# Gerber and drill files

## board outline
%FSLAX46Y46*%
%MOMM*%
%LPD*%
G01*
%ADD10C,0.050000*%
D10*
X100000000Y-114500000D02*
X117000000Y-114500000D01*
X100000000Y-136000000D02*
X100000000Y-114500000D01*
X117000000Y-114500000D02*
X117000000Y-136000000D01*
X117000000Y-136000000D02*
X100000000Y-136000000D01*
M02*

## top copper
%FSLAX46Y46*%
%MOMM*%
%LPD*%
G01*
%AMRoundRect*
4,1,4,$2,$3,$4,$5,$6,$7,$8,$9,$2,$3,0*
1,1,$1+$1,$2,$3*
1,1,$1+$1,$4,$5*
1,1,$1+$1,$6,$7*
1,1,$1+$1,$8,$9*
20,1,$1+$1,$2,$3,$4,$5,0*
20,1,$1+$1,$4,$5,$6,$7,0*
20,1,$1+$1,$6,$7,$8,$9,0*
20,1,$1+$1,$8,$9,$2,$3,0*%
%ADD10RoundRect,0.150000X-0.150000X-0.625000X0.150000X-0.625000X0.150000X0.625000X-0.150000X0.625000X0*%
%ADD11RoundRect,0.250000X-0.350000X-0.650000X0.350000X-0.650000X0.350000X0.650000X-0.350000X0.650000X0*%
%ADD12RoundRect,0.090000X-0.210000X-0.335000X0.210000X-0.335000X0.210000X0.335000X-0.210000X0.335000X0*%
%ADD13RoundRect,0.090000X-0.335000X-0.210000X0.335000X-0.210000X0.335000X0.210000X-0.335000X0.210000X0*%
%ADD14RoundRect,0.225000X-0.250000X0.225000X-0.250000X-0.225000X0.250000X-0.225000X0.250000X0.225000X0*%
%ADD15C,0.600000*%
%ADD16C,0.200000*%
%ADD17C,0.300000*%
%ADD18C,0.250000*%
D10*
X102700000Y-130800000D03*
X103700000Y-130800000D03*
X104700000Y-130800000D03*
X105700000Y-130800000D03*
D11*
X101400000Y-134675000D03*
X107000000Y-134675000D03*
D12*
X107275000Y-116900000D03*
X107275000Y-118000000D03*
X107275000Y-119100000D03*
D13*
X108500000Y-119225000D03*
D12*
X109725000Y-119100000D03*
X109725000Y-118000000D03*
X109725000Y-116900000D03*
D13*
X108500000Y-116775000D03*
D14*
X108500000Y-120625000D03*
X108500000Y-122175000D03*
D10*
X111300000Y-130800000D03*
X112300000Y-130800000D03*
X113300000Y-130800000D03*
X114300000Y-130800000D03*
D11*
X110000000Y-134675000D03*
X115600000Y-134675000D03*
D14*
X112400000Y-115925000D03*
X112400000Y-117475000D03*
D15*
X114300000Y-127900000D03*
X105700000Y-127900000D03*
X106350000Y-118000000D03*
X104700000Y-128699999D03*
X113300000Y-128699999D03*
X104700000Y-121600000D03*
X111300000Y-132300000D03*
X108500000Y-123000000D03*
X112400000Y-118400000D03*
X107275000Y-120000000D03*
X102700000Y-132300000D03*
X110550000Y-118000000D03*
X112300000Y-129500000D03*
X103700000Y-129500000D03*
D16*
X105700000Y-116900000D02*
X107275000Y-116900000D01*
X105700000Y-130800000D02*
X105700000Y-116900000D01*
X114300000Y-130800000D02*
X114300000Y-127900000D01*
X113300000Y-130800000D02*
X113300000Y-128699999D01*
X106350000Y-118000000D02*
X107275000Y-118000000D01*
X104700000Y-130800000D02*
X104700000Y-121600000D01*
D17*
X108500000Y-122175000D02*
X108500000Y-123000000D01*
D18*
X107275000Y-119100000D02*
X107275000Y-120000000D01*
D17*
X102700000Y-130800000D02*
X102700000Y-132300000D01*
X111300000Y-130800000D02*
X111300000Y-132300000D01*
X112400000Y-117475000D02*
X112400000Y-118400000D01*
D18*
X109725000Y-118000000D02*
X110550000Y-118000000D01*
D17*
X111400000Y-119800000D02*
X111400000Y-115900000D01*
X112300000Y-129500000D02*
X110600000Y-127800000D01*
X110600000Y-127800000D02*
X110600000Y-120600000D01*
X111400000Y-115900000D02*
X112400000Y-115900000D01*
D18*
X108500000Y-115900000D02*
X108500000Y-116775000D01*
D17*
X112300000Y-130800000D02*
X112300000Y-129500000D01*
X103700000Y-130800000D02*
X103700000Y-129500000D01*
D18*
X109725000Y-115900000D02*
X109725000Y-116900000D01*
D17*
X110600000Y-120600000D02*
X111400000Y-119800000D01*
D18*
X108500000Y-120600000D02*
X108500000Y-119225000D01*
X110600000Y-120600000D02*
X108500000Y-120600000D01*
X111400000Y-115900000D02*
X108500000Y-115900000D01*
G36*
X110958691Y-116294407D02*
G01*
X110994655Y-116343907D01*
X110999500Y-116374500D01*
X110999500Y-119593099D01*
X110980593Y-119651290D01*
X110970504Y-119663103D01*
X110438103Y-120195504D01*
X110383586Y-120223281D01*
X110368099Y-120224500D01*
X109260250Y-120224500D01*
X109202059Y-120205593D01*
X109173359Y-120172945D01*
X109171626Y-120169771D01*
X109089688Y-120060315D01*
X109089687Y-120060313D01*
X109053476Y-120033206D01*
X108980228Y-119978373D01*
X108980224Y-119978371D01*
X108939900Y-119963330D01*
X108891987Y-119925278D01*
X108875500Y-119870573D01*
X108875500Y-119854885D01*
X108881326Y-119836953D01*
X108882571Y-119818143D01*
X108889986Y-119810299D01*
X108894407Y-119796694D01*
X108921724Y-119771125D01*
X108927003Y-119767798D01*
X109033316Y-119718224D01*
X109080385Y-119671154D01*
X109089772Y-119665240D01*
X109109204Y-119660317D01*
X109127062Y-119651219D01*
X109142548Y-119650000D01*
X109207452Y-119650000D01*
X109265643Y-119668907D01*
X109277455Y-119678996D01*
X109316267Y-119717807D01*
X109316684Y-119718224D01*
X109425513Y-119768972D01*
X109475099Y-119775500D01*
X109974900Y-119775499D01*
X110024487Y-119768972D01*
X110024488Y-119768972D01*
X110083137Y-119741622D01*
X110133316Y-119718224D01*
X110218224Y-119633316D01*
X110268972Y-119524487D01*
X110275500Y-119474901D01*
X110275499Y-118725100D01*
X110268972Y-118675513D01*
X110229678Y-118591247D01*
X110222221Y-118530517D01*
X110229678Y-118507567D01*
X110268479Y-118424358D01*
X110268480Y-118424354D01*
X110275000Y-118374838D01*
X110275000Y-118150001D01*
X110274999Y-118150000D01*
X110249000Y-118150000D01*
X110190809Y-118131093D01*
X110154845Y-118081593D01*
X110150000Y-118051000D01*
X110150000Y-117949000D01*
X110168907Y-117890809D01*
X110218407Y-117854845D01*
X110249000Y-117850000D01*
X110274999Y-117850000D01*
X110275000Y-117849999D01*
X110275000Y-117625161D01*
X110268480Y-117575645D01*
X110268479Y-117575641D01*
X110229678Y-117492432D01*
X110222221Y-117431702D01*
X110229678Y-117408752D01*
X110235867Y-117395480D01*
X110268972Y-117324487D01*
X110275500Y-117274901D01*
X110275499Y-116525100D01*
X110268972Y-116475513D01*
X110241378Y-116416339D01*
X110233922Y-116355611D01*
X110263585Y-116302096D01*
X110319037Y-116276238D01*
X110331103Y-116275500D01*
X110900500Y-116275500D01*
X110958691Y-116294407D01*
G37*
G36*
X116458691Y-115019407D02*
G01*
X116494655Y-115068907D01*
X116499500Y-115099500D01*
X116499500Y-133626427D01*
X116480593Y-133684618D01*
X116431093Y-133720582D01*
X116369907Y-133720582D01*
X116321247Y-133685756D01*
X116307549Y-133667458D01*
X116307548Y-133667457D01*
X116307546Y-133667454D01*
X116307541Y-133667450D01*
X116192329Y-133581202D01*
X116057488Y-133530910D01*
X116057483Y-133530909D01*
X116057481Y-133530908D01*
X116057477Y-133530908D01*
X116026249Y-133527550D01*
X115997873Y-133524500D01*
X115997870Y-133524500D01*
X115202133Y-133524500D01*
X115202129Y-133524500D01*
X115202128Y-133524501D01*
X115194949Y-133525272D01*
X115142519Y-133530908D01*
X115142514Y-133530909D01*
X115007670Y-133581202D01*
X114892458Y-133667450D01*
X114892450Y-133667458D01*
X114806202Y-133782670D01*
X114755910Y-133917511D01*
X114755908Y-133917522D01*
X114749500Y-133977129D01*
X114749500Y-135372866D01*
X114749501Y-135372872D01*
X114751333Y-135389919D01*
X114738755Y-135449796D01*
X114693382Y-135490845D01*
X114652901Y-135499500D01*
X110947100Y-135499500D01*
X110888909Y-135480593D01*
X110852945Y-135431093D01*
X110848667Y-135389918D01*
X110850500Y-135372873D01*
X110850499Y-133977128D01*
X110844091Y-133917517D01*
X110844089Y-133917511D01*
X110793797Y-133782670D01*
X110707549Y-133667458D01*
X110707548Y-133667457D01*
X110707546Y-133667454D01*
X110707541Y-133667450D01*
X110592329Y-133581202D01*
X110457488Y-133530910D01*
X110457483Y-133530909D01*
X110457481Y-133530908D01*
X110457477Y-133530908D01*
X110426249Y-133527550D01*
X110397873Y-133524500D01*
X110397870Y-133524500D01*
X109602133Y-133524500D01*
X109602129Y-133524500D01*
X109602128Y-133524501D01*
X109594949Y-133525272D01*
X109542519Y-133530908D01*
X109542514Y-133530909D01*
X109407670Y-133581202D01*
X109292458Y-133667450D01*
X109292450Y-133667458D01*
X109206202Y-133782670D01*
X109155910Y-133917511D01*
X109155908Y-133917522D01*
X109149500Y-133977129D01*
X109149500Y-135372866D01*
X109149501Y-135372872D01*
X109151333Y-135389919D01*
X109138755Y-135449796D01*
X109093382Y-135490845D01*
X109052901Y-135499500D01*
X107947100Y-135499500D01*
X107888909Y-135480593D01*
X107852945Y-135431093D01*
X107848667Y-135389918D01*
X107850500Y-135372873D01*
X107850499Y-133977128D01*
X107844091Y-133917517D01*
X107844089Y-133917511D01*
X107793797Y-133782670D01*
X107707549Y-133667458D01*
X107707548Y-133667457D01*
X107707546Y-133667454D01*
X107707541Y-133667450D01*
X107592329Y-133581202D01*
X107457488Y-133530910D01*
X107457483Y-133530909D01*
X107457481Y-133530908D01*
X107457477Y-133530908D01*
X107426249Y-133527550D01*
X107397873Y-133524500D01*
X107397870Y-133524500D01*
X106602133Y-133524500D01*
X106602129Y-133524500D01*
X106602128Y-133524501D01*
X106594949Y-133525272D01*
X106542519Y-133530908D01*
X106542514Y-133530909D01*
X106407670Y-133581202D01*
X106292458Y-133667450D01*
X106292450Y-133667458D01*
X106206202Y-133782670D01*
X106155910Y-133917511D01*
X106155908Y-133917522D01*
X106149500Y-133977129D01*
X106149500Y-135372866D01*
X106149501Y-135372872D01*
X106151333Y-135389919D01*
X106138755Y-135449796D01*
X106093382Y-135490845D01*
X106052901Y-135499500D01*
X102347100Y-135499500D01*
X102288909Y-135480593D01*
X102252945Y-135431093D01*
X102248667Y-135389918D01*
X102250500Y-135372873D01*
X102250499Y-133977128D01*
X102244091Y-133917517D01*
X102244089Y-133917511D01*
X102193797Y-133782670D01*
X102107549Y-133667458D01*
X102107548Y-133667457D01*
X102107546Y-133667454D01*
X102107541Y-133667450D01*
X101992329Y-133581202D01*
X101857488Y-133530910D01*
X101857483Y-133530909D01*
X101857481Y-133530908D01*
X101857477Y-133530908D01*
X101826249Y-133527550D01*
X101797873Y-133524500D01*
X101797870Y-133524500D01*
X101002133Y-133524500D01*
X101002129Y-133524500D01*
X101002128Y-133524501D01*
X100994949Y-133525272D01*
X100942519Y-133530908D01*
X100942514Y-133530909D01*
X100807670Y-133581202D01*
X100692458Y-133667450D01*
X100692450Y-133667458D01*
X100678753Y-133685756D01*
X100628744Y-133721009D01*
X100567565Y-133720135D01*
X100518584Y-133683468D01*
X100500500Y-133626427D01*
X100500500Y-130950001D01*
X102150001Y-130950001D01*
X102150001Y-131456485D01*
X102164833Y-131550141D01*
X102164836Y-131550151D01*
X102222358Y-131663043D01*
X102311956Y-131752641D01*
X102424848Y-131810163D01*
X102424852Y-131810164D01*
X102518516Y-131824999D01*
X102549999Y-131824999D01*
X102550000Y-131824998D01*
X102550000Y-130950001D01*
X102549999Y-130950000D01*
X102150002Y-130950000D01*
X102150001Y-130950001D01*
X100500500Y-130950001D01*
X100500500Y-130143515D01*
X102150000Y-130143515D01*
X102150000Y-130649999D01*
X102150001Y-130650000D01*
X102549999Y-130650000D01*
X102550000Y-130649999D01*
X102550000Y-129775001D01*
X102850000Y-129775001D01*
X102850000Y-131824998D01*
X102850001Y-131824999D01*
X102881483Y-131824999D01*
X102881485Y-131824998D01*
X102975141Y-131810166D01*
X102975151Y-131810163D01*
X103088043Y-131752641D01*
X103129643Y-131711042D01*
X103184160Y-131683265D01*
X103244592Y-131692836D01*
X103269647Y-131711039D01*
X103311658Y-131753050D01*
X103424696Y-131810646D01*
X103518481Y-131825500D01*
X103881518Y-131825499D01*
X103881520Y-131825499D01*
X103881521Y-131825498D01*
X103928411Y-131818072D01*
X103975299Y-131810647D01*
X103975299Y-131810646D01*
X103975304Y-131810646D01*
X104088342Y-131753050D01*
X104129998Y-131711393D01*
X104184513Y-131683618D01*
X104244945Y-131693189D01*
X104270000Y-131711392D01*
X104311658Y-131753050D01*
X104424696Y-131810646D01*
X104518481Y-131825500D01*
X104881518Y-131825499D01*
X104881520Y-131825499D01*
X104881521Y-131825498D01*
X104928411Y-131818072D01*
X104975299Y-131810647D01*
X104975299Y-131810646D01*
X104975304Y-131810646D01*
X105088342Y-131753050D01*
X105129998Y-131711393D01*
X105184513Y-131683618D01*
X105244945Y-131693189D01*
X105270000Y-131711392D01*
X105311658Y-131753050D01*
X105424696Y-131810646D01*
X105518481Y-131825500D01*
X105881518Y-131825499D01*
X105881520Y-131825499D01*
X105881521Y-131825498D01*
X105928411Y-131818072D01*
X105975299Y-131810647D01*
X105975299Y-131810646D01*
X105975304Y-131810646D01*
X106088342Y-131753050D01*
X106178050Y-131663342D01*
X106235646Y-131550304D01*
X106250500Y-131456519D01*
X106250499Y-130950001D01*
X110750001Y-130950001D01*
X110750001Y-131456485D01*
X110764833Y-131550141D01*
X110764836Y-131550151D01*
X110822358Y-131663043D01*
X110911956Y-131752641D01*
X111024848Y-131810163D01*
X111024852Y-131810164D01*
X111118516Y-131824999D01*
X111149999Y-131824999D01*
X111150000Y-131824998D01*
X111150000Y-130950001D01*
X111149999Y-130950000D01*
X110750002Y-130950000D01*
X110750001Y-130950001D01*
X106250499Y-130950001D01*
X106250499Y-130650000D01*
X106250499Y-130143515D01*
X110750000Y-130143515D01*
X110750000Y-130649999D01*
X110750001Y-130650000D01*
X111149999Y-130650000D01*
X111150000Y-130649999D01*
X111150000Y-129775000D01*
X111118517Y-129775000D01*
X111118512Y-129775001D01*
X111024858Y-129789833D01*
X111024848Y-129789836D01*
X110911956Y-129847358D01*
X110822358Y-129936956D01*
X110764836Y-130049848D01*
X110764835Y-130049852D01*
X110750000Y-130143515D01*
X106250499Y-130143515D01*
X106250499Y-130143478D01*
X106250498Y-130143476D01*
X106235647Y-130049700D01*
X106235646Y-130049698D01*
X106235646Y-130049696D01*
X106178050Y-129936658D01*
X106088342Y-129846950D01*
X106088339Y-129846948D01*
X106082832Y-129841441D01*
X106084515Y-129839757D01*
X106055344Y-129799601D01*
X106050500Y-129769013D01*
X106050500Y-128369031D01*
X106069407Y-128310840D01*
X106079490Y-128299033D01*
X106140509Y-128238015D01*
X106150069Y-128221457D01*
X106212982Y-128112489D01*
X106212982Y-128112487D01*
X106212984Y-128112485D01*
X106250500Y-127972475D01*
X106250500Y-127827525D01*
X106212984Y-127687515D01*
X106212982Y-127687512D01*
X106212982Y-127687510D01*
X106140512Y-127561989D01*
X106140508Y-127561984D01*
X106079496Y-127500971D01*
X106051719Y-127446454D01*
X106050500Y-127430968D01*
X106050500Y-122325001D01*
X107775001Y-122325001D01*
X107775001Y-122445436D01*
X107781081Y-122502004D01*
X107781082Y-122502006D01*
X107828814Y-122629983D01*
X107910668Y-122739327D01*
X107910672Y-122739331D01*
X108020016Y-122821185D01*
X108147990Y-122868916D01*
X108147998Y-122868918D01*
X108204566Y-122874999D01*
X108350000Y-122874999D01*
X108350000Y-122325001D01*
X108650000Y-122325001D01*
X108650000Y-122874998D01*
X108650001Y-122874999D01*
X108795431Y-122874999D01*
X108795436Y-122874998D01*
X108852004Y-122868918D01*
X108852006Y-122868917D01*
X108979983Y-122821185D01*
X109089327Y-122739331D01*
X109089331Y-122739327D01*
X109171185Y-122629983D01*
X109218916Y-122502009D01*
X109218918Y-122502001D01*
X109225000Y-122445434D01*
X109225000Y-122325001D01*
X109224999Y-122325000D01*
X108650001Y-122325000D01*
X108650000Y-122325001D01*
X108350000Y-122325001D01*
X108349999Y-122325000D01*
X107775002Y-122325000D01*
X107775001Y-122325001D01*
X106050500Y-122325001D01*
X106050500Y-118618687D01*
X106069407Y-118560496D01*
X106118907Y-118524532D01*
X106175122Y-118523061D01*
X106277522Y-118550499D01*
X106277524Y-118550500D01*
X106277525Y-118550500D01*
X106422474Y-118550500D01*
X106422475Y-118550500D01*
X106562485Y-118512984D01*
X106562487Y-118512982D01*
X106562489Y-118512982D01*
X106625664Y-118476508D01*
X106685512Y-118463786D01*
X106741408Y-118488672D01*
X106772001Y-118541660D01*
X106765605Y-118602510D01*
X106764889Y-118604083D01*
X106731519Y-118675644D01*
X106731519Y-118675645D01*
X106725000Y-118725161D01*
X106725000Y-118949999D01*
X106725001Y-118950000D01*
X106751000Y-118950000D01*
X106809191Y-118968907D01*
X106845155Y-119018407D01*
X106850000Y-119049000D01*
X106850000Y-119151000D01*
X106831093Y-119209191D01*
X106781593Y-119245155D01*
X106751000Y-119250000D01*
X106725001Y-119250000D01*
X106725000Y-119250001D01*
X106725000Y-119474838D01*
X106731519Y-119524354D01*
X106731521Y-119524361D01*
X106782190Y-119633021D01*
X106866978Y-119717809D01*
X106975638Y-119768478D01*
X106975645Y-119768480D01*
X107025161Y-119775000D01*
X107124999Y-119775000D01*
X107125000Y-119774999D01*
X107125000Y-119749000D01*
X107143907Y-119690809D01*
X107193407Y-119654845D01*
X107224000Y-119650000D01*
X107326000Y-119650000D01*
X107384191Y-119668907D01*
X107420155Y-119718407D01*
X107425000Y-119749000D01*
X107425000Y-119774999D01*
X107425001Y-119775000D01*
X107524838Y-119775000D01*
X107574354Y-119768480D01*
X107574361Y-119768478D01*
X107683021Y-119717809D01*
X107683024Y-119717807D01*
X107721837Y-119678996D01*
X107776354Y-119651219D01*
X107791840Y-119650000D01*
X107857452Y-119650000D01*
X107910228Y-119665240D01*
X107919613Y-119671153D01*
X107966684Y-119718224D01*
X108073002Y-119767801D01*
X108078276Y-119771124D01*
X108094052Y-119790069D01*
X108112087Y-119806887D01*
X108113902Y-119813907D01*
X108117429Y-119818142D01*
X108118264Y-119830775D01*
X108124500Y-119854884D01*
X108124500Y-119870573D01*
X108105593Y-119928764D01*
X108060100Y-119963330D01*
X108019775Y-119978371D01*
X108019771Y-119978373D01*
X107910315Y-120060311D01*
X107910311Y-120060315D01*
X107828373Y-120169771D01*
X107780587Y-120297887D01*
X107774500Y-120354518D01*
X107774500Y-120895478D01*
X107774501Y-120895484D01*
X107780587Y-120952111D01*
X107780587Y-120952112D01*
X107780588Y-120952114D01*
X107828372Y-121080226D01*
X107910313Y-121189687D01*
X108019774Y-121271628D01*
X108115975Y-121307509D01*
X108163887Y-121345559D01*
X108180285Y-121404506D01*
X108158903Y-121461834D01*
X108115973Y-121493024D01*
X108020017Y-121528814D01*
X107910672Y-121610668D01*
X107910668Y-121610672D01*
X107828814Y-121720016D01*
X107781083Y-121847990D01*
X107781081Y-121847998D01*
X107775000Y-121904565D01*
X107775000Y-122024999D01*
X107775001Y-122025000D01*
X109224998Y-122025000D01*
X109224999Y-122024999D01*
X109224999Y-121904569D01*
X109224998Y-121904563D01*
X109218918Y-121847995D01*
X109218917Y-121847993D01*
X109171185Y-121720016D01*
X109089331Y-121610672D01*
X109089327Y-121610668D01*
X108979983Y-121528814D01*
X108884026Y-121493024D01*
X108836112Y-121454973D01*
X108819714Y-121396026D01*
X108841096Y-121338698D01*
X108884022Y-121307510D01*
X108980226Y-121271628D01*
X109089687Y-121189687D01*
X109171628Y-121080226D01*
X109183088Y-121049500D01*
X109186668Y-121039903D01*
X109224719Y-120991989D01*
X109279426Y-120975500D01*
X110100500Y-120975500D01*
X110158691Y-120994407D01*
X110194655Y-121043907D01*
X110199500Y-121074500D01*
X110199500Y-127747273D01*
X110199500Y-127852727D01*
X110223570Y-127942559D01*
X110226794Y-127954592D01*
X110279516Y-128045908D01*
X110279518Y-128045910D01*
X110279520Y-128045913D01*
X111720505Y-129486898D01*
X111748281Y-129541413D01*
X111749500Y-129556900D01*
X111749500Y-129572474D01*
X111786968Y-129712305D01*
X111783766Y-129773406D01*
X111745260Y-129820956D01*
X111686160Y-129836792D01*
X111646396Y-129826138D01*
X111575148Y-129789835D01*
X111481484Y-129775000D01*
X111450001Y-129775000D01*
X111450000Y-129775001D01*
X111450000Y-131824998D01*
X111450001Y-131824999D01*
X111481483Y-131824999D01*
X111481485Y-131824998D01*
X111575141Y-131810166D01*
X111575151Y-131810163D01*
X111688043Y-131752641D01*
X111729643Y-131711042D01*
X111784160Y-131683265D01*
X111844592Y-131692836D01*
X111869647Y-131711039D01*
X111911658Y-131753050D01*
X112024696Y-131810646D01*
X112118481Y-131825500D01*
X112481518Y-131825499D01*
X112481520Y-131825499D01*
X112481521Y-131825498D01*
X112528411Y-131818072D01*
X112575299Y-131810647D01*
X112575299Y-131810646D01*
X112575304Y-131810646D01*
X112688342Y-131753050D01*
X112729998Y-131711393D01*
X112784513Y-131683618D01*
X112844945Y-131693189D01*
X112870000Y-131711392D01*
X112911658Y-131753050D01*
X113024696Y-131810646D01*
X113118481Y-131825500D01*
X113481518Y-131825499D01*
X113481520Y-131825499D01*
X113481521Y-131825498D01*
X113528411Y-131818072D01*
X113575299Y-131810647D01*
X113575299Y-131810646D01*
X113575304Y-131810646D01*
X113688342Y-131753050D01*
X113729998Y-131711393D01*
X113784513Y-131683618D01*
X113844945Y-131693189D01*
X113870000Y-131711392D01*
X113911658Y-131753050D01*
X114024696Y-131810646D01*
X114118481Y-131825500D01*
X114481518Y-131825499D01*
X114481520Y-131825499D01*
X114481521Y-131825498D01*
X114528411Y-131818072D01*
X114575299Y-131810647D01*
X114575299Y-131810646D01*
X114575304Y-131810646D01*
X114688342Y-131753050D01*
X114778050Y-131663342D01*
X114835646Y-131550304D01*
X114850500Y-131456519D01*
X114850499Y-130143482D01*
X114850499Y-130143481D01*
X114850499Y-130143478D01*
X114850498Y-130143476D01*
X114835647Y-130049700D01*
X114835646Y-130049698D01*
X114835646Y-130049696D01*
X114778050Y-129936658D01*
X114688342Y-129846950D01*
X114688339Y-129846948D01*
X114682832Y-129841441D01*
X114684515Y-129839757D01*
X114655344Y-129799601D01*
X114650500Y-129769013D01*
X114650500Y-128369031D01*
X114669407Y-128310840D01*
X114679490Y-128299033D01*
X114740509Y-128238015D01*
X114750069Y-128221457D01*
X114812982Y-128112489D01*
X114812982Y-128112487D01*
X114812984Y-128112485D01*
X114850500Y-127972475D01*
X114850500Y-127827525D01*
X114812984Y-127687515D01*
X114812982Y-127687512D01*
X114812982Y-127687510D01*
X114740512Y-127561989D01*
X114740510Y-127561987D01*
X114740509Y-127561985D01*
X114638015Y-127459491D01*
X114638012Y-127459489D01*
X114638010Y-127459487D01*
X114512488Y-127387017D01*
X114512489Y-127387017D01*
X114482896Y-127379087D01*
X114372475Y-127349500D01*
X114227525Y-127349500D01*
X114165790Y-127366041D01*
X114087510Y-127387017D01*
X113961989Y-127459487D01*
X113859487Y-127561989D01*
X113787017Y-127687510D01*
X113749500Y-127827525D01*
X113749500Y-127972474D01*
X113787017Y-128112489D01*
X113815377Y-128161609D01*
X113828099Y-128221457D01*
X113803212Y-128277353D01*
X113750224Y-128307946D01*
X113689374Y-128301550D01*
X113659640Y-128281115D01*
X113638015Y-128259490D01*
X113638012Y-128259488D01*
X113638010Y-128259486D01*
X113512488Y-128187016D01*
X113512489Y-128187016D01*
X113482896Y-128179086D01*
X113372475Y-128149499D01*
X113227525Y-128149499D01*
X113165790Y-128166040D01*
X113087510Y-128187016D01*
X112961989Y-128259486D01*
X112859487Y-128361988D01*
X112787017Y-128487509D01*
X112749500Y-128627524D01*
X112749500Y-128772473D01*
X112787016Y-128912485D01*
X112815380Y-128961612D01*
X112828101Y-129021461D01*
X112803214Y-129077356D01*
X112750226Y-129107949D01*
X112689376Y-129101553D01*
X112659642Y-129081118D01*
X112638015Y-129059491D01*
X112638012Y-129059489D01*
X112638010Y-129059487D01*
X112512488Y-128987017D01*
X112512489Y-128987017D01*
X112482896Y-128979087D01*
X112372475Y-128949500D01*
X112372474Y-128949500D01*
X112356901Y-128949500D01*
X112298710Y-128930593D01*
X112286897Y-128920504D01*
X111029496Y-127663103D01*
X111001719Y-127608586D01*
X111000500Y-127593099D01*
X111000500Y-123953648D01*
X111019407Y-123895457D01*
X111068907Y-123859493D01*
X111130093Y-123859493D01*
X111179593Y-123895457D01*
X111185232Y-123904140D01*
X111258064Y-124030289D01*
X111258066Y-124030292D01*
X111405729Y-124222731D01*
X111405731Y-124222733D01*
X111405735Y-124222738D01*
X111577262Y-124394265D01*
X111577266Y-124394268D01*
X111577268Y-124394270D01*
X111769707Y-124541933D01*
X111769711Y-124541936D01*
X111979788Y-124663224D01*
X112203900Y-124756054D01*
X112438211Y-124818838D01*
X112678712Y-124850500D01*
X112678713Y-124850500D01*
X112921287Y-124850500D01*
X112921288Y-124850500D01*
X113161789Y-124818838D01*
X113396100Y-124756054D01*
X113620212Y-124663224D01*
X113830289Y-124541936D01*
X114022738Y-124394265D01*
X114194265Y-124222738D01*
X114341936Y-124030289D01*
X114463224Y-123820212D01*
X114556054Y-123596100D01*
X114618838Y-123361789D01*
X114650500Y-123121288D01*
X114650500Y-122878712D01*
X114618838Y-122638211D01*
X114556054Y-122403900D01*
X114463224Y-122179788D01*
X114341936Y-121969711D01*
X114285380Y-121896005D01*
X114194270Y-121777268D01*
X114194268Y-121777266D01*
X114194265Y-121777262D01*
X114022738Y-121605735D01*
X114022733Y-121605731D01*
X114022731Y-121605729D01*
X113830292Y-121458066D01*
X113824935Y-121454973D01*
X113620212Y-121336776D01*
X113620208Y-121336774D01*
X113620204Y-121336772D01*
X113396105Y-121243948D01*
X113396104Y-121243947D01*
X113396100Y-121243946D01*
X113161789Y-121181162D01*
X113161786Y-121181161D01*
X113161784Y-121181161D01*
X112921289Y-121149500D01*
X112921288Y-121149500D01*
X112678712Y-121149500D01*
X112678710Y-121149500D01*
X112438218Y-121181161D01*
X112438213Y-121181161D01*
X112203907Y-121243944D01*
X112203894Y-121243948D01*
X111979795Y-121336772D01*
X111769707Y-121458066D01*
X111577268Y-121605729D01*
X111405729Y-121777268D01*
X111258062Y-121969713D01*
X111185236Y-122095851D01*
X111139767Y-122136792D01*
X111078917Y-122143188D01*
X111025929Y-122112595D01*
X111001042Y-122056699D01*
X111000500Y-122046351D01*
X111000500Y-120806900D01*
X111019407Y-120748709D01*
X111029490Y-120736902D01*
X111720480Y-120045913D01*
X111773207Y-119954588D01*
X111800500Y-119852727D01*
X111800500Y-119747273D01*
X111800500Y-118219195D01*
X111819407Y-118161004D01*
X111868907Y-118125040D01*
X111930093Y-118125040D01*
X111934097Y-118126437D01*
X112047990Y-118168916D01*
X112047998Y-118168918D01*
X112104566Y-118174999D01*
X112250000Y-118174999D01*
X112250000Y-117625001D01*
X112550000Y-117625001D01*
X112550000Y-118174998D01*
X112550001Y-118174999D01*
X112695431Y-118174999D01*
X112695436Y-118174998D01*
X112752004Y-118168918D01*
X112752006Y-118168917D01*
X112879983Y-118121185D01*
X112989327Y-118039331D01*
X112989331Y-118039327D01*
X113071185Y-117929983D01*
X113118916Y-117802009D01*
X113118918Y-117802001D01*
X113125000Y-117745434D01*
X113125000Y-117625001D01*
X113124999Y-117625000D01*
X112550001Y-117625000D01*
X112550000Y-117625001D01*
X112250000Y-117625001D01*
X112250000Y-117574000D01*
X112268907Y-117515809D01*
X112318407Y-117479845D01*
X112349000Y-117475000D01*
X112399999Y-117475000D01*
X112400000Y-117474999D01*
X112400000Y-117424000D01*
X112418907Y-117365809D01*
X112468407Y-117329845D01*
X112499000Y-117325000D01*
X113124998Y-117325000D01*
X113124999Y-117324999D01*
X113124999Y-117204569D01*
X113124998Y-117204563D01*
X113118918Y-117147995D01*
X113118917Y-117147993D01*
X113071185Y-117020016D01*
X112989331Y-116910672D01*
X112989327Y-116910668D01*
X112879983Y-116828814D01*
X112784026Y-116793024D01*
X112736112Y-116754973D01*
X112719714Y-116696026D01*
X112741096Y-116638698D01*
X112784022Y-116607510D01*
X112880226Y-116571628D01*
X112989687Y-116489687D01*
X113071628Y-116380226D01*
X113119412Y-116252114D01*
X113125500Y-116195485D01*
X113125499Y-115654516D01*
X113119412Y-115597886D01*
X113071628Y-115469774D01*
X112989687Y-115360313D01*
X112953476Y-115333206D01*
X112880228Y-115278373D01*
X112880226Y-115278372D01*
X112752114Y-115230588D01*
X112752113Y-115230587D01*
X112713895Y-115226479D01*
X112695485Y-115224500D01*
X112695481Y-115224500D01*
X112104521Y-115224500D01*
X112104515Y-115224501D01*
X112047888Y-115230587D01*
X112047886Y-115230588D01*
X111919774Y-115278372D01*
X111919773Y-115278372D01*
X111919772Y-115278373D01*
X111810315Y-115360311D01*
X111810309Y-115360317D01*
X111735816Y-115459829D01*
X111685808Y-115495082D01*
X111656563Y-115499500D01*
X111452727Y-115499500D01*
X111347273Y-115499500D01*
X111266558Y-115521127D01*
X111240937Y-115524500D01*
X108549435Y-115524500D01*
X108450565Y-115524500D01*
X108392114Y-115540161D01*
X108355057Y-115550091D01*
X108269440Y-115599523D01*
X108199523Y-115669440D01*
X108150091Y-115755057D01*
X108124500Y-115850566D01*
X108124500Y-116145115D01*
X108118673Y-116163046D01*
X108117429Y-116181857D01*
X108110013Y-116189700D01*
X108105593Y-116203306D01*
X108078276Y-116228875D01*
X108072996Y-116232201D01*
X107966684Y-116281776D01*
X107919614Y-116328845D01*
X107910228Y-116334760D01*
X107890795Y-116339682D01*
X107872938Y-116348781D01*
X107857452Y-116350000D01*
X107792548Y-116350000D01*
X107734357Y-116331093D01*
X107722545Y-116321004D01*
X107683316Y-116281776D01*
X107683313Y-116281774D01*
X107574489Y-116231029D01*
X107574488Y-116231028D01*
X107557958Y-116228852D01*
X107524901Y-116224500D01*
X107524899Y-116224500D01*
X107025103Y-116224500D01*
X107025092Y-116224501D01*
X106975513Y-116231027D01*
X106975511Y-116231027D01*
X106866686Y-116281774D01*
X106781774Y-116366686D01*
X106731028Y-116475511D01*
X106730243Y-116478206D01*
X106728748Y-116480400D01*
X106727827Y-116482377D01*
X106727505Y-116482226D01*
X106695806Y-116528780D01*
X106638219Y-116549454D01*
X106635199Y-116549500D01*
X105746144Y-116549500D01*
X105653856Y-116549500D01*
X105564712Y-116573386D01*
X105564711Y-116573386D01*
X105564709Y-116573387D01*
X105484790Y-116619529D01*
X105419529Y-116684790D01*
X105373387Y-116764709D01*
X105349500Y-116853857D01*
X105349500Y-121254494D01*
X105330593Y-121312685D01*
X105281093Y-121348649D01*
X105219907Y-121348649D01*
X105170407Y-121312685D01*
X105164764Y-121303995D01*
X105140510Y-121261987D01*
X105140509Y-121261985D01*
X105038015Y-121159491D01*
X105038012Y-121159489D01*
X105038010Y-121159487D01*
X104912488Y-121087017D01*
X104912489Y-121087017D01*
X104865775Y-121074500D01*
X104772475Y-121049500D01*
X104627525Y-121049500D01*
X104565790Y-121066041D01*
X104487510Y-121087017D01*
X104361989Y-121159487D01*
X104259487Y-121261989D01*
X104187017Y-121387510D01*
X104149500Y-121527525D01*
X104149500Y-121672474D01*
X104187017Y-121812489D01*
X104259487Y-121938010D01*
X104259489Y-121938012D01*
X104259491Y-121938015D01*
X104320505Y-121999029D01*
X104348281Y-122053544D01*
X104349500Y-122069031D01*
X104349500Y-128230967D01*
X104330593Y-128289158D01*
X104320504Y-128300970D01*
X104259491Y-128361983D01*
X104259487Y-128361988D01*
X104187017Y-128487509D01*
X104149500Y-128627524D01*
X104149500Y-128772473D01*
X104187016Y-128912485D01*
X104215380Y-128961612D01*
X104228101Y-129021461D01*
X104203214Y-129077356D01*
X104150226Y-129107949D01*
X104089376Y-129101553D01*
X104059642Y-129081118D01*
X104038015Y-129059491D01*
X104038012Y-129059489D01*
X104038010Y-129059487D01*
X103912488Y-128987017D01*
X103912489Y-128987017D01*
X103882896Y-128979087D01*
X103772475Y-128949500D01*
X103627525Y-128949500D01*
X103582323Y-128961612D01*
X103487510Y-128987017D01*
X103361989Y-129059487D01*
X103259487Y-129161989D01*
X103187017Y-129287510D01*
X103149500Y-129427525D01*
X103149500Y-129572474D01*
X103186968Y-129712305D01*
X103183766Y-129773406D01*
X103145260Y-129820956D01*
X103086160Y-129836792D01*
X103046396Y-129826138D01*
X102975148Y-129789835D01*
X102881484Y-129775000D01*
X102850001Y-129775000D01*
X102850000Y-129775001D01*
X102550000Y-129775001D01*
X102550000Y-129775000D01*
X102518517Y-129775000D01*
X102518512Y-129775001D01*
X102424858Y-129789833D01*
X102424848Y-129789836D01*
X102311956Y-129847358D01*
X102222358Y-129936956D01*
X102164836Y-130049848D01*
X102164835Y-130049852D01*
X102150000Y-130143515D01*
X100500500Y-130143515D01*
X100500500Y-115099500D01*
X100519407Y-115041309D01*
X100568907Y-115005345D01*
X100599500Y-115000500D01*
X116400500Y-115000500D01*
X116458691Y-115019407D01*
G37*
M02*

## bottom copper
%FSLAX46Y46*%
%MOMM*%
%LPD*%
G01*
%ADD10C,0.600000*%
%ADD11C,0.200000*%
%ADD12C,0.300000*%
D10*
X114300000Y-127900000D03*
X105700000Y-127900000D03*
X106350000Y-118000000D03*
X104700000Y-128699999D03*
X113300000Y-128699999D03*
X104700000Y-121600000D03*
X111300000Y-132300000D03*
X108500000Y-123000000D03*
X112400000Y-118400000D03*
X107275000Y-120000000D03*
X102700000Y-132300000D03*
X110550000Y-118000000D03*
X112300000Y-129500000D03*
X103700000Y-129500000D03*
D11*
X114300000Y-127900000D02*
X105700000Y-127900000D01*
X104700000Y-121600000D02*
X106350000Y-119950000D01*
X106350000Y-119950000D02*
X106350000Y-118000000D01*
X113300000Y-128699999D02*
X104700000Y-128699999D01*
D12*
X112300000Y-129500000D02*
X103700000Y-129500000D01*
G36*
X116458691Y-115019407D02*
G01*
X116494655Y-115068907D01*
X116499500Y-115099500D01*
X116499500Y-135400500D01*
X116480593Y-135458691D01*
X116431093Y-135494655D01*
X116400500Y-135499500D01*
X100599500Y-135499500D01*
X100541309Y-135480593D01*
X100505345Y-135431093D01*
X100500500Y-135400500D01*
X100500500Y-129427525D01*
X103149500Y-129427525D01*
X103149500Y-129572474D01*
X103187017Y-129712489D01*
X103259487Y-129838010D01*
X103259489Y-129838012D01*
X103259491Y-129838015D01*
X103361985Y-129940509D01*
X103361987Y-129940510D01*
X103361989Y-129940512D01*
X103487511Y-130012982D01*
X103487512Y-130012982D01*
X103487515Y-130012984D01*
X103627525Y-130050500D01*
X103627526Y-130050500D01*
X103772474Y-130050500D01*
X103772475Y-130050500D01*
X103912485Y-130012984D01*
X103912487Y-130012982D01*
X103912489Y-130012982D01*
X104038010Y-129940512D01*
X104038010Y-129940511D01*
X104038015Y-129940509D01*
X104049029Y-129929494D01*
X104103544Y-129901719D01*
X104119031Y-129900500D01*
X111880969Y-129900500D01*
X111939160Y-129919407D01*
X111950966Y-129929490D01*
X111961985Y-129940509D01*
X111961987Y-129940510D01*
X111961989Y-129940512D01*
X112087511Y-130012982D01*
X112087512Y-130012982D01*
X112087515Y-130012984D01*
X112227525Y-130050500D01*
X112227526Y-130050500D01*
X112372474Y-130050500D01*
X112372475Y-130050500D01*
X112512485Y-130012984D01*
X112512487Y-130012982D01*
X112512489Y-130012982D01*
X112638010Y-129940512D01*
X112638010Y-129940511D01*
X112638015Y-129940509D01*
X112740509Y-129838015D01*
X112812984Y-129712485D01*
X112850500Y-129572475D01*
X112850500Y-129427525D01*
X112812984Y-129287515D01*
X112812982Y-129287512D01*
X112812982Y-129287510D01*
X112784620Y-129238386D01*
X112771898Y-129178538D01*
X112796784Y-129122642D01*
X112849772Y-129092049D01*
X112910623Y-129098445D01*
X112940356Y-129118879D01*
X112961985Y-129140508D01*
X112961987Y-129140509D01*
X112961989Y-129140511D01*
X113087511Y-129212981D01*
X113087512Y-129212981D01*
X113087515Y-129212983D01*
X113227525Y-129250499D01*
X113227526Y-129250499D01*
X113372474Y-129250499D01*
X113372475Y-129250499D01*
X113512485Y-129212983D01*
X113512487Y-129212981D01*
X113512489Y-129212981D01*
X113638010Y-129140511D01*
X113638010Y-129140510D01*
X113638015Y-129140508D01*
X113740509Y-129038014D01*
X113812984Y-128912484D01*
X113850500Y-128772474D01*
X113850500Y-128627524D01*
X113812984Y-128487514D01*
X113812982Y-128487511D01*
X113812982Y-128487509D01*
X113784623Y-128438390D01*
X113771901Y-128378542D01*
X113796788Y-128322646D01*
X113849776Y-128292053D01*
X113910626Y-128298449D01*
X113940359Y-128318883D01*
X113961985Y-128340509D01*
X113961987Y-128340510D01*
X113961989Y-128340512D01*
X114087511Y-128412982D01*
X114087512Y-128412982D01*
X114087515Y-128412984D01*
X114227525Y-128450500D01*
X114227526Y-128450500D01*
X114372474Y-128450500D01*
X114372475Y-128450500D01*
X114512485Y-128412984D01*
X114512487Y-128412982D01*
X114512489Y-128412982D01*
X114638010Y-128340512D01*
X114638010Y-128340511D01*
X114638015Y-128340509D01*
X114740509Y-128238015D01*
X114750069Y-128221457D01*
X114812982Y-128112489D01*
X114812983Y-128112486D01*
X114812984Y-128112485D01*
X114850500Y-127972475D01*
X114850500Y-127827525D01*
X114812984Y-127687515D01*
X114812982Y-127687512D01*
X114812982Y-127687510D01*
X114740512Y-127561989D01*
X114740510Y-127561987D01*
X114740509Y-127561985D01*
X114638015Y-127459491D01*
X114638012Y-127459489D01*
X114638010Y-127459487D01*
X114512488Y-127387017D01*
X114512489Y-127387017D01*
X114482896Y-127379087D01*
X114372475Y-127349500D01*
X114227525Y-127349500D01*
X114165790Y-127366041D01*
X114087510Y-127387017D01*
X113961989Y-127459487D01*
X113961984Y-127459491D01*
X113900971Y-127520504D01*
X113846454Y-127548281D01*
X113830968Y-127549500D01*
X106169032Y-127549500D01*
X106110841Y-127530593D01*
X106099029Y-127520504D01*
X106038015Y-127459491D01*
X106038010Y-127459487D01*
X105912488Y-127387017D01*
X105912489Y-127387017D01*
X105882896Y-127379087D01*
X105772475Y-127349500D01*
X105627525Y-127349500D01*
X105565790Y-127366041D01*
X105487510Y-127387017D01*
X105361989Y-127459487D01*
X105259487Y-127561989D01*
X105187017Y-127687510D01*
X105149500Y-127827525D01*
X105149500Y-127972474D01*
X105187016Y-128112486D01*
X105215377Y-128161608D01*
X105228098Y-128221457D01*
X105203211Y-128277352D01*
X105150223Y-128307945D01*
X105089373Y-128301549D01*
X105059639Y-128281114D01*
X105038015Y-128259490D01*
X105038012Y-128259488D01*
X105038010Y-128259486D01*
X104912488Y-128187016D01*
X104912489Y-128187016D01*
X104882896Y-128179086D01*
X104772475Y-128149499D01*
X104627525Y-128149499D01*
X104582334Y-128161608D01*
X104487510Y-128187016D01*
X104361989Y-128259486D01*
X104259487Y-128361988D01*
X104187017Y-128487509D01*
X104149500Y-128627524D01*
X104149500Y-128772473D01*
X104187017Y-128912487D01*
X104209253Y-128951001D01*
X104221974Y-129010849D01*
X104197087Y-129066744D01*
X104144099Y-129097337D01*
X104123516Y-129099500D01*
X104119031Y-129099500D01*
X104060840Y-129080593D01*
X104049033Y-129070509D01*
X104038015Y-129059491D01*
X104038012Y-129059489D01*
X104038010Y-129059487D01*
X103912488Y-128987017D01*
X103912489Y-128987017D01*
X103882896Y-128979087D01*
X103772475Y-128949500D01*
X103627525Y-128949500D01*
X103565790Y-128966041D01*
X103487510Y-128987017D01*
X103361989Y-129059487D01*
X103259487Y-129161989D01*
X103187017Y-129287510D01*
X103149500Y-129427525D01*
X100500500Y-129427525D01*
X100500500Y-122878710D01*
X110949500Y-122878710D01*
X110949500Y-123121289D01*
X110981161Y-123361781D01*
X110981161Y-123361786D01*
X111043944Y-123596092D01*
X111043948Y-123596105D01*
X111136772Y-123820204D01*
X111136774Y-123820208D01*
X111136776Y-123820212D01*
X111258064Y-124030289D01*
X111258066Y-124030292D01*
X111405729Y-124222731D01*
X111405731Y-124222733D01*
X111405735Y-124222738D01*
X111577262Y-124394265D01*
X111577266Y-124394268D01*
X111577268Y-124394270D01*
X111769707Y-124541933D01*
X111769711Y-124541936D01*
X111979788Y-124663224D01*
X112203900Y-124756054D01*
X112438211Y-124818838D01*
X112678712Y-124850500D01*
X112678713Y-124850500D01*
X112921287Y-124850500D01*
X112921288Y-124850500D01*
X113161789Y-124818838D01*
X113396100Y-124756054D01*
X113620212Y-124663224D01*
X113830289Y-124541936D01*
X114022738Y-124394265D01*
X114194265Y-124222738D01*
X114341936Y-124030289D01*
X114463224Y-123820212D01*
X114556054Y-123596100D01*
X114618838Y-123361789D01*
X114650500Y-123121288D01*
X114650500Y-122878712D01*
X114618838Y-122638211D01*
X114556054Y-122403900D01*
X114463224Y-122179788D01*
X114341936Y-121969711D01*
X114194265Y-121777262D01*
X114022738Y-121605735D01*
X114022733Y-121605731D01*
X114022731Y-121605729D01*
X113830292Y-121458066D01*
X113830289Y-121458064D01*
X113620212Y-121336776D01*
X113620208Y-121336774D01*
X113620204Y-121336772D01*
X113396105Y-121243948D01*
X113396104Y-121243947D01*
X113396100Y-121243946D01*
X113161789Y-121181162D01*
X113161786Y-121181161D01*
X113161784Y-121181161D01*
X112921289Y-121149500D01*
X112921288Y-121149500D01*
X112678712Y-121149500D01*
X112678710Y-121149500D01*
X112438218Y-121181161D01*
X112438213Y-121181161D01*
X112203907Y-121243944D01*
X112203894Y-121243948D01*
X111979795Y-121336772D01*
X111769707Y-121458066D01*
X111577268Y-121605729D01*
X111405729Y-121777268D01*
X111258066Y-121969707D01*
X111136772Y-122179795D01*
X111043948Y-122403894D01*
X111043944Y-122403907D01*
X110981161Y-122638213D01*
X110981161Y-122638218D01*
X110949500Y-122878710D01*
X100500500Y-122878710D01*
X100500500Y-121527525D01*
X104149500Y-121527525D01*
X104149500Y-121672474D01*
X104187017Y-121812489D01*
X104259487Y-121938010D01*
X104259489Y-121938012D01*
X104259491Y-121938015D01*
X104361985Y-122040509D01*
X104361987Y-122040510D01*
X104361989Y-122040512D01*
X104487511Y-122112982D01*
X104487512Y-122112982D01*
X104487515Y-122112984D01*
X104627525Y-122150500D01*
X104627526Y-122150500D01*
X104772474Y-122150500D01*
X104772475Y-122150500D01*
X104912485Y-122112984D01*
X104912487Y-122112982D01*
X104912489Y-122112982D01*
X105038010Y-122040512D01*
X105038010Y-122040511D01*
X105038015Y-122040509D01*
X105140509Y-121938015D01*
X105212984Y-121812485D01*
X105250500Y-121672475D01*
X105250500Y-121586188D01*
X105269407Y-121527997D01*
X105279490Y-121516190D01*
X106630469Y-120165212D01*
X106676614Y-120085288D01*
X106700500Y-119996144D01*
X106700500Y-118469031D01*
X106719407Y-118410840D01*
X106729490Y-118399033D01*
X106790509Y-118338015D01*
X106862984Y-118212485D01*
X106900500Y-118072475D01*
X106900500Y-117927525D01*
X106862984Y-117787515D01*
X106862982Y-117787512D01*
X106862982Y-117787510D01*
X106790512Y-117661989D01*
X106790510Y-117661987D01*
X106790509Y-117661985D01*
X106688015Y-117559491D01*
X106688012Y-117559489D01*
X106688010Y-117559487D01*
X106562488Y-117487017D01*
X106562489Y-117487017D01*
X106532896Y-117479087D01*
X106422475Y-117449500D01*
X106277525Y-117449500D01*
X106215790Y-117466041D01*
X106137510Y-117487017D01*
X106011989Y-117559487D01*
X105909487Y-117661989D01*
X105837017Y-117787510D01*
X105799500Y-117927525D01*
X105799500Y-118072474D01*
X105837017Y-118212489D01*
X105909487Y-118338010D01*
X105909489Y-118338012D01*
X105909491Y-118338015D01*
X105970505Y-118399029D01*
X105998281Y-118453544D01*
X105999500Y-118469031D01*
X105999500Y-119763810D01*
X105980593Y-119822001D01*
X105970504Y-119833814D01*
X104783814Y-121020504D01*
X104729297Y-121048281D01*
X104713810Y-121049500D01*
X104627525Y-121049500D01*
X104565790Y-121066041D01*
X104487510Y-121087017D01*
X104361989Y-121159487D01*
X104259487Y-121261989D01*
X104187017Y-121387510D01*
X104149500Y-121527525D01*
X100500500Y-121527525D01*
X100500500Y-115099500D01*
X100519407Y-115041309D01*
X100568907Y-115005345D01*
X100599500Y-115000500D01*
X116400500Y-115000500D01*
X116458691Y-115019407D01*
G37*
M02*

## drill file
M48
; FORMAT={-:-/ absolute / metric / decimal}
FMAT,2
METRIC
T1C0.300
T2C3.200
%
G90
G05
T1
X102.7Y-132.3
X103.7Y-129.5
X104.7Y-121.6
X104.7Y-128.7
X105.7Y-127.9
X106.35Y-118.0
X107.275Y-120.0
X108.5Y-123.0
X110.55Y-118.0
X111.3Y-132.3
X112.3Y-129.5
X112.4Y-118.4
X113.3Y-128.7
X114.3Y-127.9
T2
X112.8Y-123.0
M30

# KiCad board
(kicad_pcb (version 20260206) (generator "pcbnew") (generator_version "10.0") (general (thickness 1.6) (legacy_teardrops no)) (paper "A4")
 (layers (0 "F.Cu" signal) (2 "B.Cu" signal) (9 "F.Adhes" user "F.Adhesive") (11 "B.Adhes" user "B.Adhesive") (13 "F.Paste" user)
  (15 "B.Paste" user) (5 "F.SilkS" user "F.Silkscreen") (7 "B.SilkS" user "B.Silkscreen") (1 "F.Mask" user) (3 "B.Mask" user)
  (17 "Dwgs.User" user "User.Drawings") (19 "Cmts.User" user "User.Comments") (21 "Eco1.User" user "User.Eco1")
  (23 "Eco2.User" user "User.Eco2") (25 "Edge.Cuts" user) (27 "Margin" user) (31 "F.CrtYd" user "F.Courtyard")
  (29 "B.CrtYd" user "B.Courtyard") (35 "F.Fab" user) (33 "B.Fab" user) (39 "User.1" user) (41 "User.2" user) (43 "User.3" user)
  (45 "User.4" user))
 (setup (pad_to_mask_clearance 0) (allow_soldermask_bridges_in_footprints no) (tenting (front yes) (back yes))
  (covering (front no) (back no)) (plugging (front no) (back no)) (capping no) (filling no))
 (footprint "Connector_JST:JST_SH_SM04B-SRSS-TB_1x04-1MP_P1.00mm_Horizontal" (layer "F.Cu") (at 104.2 132.8)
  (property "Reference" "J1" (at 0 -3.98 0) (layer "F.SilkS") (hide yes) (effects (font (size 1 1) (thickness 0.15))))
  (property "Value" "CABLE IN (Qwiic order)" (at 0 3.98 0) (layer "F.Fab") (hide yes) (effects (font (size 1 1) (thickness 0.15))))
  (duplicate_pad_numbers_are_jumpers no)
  (pad "1" smd roundrect (at -1.5 -2) (size 0.6 1.55) (layers "F.Cu" "F.Mask" "F.Paste") (roundrect_rratio 0.25) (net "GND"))
  (pad "2" smd roundrect (at -0.5 -2) (size 0.6 1.55) (layers "F.Cu" "F.Mask" "F.Paste") (roundrect_rratio 0.25) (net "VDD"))
  (pad "3" smd roundrect (at 0.5 -2) (size 0.6 1.55) (layers "F.Cu" "F.Mask" "F.Paste") (roundrect_rratio 0.25) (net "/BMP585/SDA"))
  (pad "4" smd roundrect (at 1.5 -2) (size 0.6 1.55) (layers "F.Cu" "F.Mask" "F.Paste") (roundrect_rratio 0.25) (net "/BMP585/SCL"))
  (pad "MP" smd roundrect (at -2.8 1.875) (size 1.2 1.8) (layers "F.Cu" "F.Mask" "F.Paste") (roundrect_rratio 0.208333))
  (pad "MP" smd roundrect (at 2.8 1.875) (size 1.2 1.8) (layers "F.Cu" "F.Mask" "F.Paste") (roundrect_rratio 0.208333)))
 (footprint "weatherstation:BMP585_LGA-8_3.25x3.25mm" (layer "F.Cu") (at 108.5 118)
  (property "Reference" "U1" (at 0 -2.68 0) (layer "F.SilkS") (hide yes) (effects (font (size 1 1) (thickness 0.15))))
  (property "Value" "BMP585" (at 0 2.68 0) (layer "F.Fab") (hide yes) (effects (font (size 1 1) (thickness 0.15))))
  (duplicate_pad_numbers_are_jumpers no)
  (pad "1" smd roundrect (at -1.225 -1.1) (size 0.6 0.85) (layers "F.Cu" "F.Mask" "F.Paste") (roundrect_rratio 0.15) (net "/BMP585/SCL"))
  (pad "2" smd roundrect (at -1.225 0) (size 0.6 0.85) (layers "F.Cu" "F.Mask" "F.Paste") (roundrect_rratio 0.15) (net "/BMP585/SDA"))
  (pad "3" smd roundrect (at -1.225 1.1) (size 0.6 0.85) (layers "F.Cu" "F.Mask" "F.Paste") (roundrect_rratio 0.15) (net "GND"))
  (pad "4" smd roundrect (at 0 1.225) (size 0.85 0.6) (layers "F.Cu" "F.Mask" "F.Paste") (roundrect_rratio 0.15) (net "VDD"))
  (pad "5" smd roundrect (at 1.225 1.1) (size 0.6 0.85) (layers "F.Cu" "F.Mask" "F.Paste") (roundrect_rratio 0.15)
   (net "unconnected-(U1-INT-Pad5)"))
  (pad "6" smd roundrect (at 1.225 0) (size 0.6 0.85) (layers "F.Cu" "F.Mask" "F.Paste") (roundrect_rratio 0.15) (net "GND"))
  (pad "7" smd roundrect (at 1.225 -1.1) (size 0.6 0.85) (layers "F.Cu" "F.Mask" "F.Paste") (roundrect_rratio 0.15) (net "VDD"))
  (pad "8" smd roundrect (at 0 -1.225) (size 0.85 0.6) (layers "F.Cu" "F.Mask" "F.Paste") (roundrect_rratio 0.15) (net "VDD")))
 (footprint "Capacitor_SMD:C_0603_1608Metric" (layer "F.Cu") (at 108.5 121.4 -90)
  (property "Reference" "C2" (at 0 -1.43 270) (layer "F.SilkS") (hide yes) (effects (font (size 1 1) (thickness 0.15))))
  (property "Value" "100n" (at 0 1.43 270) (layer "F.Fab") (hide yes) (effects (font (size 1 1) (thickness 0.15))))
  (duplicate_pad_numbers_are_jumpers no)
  (pad "1" smd roundrect (at -0.775 0 270) (size 0.9 0.95) (layers "F.Cu" "F.Mask" "F.Paste") (roundrect_rratio 0.25) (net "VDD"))
  (pad "2" smd roundrect (at 0.775 0 270) (size 0.9 0.95) (layers "F.Cu" "F.Mask" "F.Paste") (roundrect_rratio 0.25) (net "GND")))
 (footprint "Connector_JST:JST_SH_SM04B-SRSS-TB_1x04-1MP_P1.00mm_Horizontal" (layer "F.Cu") (at 112.8 132.8)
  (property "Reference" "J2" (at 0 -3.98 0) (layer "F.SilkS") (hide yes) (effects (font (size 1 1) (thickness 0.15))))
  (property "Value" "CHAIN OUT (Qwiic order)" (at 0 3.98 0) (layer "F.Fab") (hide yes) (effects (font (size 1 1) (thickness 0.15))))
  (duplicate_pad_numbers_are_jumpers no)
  (pad "1" smd roundrect (at -1.5 -2) (size 0.6 1.55) (layers "F.Cu" "F.Mask" "F.Paste") (roundrect_rratio 0.25) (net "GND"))
  (pad "2" smd roundrect (at -0.5 -2) (size 0.6 1.55) (layers "F.Cu" "F.Mask" "F.Paste") (roundrect_rratio 0.25) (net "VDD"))
  (pad "3" smd roundrect (at 0.5 -2) (size 0.6 1.55) (layers "F.Cu" "F.Mask" "F.Paste") (roundrect_rratio 0.25) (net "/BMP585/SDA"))
  (pad "4" smd roundrect (at 1.5 -2) (size 0.6 1.55) (layers "F.Cu" "F.Mask" "F.Paste") (roundrect_rratio 0.25) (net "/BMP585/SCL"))
  (pad "MP" smd roundrect (at -2.8 1.875) (size 1.2 1.8) (layers "F.Cu" "F.Mask" "F.Paste") (roundrect_rratio 0.208333))
  (pad "MP" smd roundrect (at 2.8 1.875) (size 1.2 1.8) (layers "F.Cu" "F.Mask" "F.Paste") (roundrect_rratio 0.208333)))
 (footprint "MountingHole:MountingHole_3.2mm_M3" (layer "F.Cu") (at 112.8 123)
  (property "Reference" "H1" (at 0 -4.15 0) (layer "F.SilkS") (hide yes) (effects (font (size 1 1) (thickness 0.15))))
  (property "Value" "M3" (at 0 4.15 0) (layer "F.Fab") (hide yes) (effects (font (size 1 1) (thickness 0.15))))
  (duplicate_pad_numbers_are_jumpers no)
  (pad "" np_thru_hole circle (at 0 0) (size 3.2 3.2) (drill 3.2) (layers "*.Cu" "*.Mask")))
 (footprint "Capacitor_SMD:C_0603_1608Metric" (layer "F.Cu") (at 112.4 116.7 -90)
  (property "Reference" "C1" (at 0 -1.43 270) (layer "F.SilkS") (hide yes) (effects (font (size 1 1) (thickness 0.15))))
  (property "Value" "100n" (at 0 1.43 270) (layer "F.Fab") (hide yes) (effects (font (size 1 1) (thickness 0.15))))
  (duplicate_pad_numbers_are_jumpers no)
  (pad "1" smd roundrect (at -0.775 0 270) (size 0.9 0.95) (layers "F.Cu" "F.Mask" "F.Paste") (roundrect_rratio 0.25) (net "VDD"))
  (pad "2" smd roundrect (at 0.775 0 270) (size 0.9 0.95) (layers "F.Cu" "F.Mask" "F.Paste") (roundrect_rratio 0.25) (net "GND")))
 (gr_line (start 100 114.5) (end 117 114.5) (stroke (width 0.05) (type default)) (layer "Edge.Cuts"))
 (gr_line (start 100 136) (end 100 114.5) (stroke (width 0.05) (type default)) (layer "Edge.Cuts"))
 (gr_line (start 117 114.5) (end 117 136) (stroke (width 0.05) (type default)) (layer "Edge.Cuts"))
 (gr_line (start 117 136) (end 100 136) (stroke (width 0.05) (type default)) (layer "Edge.Cuts"))
 (segment (start 105.7 116.9) (end 107.275 116.9) (width 0.2) (layer "F.Cu") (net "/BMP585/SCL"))
 (segment (start 105.7 130.8) (end 105.7 116.9) (width 0.2) (layer "F.Cu") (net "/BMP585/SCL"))
 (segment (start 114.3 130.8) (end 114.3 127.9) (width 0.2) (layer "F.Cu") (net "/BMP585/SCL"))
 (via (at 114.3 127.9) (size 0.6) (drill 0.3) (layers "F.Cu" "B.Cu") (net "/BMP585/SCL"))
 (via (at 105.7 127.9) (size 0.6) (drill 0.3) (layers "F.Cu" "B.Cu") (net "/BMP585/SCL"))
 (segment (start 114.3 127.9) (end 105.7 127.9) (width 0.2) (layer "B.Cu") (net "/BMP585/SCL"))
 (segment (start 113.3 130.8) (end 113.3 128.699999) (width 0.2) (layer "F.Cu") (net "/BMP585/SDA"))
 (segment (start 106.35 118) (end 107.275 118) (width 0.2) (layer "F.Cu") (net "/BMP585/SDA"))
 (segment (start 104.7 130.8) (end 104.7 121.6) (width 0.2) (layer "F.Cu") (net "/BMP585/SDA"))
 (via (at 106.35 118) (size 0.6) (drill 0.3) (layers "F.Cu" "B.Cu") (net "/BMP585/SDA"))
 (via (at 104.7 128.699999) (size 0.6) (drill 0.3) (layers "F.Cu" "B.Cu") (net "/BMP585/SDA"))
 (via (at 113.3 128.699999) (size 0.6) (drill 0.3) (layers "F.Cu" "B.Cu") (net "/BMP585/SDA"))
 (via (at 104.7 121.6) (size 0.6) (drill 0.3) (layers "F.Cu" "B.Cu") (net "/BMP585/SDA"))
 (segment (start 104.7 121.6) (end 106.35 119.95) (width 0.2) (layer "B.Cu") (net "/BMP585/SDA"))
 (segment (start 106.35 119.95) (end 106.35 118) (width 0.2) (layer "B.Cu") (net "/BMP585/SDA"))
 (segment (start 113.3 128.699999) (end 104.7 128.699999) (width 0.2) (layer "B.Cu") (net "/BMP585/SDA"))
 (segment (start 108.5 122.175) (end 108.5 123) (width 0.3) (layer "F.Cu") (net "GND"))
 (segment (start 107.275 119.1) (end 107.275 120) (width 0.25) (layer "F.Cu") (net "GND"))
 (segment (start 102.7 130.8) (end 102.7 132.3) (width 0.3) (layer "F.Cu") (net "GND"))
 (segment (start 111.3 130.8) (end 111.3 132.3) (width 0.3) (layer "F.Cu") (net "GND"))
 (segment (start 112.4 117.475) (end 112.4 118.4) (width 0.3) (layer "F.Cu") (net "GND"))
 (segment (start 109.725 118) (end 110.55 118) (width 0.25) (layer "F.Cu") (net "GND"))
 (via (at 111.3 132.3) (size 0.6) (drill 0.3) (layers "F.Cu" "B.Cu") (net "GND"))
 (via (at 108.5 123) (size 0.6) (drill 0.3) (layers "F.Cu" "B.Cu") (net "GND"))
 (via (at 112.4 118.4) (size 0.6) (drill 0.3) (layers "F.Cu" "B.Cu") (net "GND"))
 (via (at 107.275 120) (size 0.6) (drill 0.3) (layers "F.Cu" "B.Cu") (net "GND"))
 (via (at 102.7 132.3) (size 0.6) (drill 0.3) (layers "F.Cu" "B.Cu") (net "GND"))
 (via (at 110.55 118) (size 0.6) (drill 0.3) (layers "F.Cu" "B.Cu") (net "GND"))
 (segment (start 111.4 119.8) (end 111.4 115.9) (width 0.3) (layer "F.Cu") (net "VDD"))
 (segment (start 112.3 129.5) (end 110.6 127.8) (width 0.3) (layer "F.Cu") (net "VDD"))
 (segment (start 110.6 127.8) (end 110.6 120.6) (width 0.3) (layer "F.Cu") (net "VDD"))
 (segment (start 111.4 115.9) (end 112.4 115.9) (width 0.3) (layer "F.Cu") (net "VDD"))
 (segment (start 108.5 115.9) (end 108.5 116.775) (width 0.25) (layer "F.Cu") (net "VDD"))
 (segment (start 112.3 130.8) (end 112.3 129.5) (width 0.3) (layer "F.Cu") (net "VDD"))
 (segment (start 103.7 130.8) (end 103.7 129.5) (width 0.3) (layer "F.Cu") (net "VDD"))
 (segment (start 109.725 115.9) (end 109.725 116.9) (width 0.25) (layer "F.Cu") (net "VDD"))
 (segment (start 110.6 120.6) (end 111.4 119.8) (width 0.3) (layer "F.Cu") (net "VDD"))
 (segment (start 108.5 120.6) (end 108.5 119.225) (width 0.25) (layer "F.Cu") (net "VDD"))
 (segment (start 110.6 120.6) (end 108.5 120.6) (width 0.25) (layer "F.Cu") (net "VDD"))
 (segment (start 111.4 115.9) (end 108.5 115.9) (width 0.25) (layer "F.Cu") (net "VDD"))
 (via (at 112.3 129.5) (size 0.6) (drill 0.3) (layers "F.Cu" "B.Cu") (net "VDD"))
 (via (at 103.7 129.5) (size 0.6) (drill 0.3) (layers "F.Cu" "B.Cu") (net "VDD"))
 (segment (start 112.3 129.5) (end 103.7 129.5) (width 0.3) (layer "B.Cu") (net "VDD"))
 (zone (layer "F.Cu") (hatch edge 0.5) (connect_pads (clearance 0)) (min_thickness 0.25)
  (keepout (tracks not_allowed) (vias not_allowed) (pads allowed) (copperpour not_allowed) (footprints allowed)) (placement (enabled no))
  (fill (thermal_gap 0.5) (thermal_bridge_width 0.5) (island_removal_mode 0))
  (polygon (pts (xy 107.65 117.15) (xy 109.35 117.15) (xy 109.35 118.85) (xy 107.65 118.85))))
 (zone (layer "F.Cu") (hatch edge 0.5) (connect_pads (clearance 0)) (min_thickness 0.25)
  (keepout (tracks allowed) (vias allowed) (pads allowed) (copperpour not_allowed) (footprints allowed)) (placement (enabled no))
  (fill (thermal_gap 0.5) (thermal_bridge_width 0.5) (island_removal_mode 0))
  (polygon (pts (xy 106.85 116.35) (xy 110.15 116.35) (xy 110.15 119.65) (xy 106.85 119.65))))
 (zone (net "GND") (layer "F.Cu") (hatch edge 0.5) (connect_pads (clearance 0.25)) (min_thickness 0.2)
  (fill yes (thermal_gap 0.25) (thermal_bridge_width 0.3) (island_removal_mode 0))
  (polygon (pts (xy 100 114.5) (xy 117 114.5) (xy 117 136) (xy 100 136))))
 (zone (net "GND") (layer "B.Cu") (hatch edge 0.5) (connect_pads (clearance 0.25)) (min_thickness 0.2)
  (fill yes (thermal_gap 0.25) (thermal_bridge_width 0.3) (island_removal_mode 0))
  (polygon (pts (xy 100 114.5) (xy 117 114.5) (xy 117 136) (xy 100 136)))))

